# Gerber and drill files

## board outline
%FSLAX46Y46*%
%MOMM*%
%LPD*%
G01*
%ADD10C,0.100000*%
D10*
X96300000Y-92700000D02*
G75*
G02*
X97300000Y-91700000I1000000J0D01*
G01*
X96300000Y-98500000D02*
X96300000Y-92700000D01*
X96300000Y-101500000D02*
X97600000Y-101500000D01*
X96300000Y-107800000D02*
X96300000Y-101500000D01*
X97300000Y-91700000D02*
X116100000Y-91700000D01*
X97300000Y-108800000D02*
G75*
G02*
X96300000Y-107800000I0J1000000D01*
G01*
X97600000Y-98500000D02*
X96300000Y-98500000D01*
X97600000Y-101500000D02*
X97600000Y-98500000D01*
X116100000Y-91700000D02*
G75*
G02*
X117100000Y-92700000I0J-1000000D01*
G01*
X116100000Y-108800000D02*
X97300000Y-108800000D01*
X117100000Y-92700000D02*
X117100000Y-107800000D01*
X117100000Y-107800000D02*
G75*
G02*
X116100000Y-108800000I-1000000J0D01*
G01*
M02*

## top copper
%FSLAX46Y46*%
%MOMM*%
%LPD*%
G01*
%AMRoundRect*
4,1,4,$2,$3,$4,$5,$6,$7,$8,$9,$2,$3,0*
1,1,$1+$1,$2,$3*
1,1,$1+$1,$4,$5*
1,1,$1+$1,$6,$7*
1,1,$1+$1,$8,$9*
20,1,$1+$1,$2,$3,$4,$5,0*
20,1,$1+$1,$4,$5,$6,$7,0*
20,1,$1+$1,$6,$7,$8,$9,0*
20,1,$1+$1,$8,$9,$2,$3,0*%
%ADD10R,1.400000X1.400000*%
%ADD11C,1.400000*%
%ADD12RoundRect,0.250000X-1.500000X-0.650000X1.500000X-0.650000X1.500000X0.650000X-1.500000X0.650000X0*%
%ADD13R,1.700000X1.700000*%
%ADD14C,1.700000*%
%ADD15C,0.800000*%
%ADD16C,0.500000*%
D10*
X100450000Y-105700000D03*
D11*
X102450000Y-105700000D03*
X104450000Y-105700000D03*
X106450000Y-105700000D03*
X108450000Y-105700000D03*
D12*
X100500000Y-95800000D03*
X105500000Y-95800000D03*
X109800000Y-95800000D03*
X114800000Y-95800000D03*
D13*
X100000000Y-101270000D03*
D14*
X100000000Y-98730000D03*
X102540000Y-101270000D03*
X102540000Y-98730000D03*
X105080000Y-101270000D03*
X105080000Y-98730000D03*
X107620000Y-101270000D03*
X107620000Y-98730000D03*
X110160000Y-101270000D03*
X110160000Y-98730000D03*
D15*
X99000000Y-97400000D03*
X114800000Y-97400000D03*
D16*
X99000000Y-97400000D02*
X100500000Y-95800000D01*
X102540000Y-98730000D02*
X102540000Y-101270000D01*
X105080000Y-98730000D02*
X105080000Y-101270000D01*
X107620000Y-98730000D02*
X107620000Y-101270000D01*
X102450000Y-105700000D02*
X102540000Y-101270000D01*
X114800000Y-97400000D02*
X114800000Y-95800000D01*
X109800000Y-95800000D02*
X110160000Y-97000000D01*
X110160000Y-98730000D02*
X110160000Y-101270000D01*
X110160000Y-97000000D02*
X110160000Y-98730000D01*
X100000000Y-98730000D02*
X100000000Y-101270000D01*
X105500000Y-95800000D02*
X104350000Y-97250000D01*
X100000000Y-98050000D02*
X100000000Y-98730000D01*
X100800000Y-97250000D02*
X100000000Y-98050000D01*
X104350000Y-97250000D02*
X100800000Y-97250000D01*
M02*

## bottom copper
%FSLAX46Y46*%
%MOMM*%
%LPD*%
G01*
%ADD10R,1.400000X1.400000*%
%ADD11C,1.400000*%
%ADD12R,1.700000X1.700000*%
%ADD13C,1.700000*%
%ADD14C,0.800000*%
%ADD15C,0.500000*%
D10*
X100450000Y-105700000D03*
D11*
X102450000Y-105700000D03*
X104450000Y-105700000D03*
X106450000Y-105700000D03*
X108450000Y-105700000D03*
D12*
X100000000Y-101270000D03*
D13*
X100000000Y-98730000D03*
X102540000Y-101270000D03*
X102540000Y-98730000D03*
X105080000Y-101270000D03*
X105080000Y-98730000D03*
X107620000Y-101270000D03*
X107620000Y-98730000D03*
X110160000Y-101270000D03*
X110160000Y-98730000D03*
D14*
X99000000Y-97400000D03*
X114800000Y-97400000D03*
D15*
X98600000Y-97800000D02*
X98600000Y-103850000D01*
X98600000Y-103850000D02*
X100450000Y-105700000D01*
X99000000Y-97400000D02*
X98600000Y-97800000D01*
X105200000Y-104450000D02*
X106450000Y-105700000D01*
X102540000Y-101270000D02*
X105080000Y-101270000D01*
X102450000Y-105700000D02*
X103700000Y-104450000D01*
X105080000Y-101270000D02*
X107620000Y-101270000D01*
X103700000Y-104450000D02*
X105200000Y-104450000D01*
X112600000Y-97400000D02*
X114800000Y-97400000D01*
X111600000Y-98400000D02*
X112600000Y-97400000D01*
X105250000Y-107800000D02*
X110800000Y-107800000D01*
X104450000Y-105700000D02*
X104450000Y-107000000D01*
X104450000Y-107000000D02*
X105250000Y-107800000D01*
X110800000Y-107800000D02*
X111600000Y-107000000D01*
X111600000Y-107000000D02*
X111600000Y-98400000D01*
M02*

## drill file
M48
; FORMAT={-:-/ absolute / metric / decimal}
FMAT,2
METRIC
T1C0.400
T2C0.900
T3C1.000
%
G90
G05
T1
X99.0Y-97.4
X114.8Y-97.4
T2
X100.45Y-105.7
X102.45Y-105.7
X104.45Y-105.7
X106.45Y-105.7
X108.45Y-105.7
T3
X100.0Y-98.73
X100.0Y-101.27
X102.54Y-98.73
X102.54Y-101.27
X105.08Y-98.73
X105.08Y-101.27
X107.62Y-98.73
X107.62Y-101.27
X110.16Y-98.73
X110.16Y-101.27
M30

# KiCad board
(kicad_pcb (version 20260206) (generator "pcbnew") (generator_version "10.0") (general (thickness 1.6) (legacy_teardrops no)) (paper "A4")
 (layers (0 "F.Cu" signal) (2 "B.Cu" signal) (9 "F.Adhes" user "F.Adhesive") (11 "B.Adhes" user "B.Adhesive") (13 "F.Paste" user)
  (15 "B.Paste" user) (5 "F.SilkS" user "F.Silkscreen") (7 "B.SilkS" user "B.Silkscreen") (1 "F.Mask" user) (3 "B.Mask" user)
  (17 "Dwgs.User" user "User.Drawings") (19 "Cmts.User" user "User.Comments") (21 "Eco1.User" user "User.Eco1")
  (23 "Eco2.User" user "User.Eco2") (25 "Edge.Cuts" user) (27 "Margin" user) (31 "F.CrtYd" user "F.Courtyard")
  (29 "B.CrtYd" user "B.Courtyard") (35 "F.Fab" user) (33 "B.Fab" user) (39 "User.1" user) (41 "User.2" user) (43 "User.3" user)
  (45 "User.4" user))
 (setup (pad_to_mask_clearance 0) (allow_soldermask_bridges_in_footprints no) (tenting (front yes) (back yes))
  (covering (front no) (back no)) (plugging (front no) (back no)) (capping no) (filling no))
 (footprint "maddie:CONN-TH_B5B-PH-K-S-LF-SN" (layer "F.Cu") (at 104.45 105.7 180)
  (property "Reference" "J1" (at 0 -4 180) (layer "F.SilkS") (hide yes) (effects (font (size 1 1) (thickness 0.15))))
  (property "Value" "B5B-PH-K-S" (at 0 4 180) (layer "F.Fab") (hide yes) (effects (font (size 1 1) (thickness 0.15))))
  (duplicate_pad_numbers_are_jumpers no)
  (pad "1" thru_hole rect (at 4 0 180) (size 1.4 1.4) (drill 0.900024) (layers "*.Cu" "*.Mask") (remove_unused_layers no) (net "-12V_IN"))
  (pad "2" thru_hole circle (at 2 0 180) (size 1.4 1.4) (drill 0.900024) (layers "*.Cu" "*.Mask") (remove_unused_layers no) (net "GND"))
  (pad "3" thru_hole circle (at 0 0 180) (size 1.4 1.4) (drill 0.900024) (layers "*.Cu" "*.Mask") (remove_unused_layers no) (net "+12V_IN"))
  (pad "4" thru_hole circle (at -2 0 180) (size 1.4 1.4) (drill 0.900024) (layers "*.Cu" "*.Mask") (remove_unused_layers no) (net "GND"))
  (pad "5" thru_hole circle (at -4 0 180) (size 1.4 1.4) (drill 0.900024) (layers "*.Cu" "*.Mask") (remove_unused_layers no)
   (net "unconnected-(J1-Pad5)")))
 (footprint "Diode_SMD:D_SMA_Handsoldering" (layer "F.Cu") (at 103 95.8)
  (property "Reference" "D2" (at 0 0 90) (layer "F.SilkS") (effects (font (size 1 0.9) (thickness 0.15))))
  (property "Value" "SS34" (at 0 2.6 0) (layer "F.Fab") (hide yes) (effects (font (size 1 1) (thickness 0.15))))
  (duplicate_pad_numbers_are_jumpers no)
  (pad "1" smd roundrect (at -2.5 0) (size 3.5 1.8) (layers "F.Cu" "F.Mask" "F.Paste") (roundrect_rratio 0.1388888889) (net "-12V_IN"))
  (pad "2" smd roundrect (at 2.5 0) (size 3.5 1.8) (layers "F.Cu" "F.Mask" "F.Paste") (roundrect_rratio 0.1388888889) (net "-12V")))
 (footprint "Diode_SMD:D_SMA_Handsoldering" (layer "F.Cu") (at 112.3 95.8)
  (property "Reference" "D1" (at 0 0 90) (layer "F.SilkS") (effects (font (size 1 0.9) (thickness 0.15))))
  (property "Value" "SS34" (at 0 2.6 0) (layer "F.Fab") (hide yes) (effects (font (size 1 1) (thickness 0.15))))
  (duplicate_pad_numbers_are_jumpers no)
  (pad "1" smd roundrect (at -2.5 0) (size 3.5 1.8) (layers "F.Cu" "F.Mask" "F.Paste") (roundrect_rratio 0.1388888889) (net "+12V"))
  (pad "2" smd roundrect (at 2.5 0) (size 3.5 1.8) (layers "F.Cu" "F.Mask" "F.Paste") (roundrect_rratio 0.1388888889) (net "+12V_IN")))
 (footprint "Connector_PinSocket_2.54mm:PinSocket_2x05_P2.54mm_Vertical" (layer "B.Cu") (at 100 101.27 -90)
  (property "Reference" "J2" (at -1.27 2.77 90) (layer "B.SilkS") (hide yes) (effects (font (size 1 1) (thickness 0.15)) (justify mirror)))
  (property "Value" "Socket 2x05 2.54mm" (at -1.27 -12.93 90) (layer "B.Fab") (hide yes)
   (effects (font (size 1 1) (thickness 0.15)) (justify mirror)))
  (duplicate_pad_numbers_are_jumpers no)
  (pad "1" thru_hole rect (at 0 0 270) (size 1.7 1.7) (drill 1) (layers "*.Cu" "*.Mask") (remove_unused_layers no) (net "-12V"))
  (pad "2" thru_hole circle (at -2.54 0 270) (size 1.7 1.7) (drill 1) (layers "*.Cu" "*.Mask") (remove_unused_layers no) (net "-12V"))
  (pad "3" thru_hole circle (at 0 -2.54 270) (size 1.7 1.7) (drill 1) (layers "*.Cu" "*.Mask") (remove_unused_layers no) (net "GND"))
  (pad "4" thru_hole circle (at -2.54 -2.54 270) (size 1.7 1.7) (drill 1) (layers "*.Cu" "*.Mask") (remove_unused_layers no) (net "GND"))
  (pad "5" thru_hole circle (at 0 -5.08 270) (size 1.7 1.7) (drill 1) (layers "*.Cu" "*.Mask") (remove_unused_layers no) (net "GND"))
  (pad "6" thru_hole circle (at -2.54 -5.08 270) (size 1.7 1.7) (drill 1) (layers "*.Cu" "*.Mask") (remove_unused_layers no) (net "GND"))
  (pad "7" thru_hole circle (at 0 -7.62 270) (size 1.7 1.7) (drill 1) (layers "*.Cu" "*.Mask") (remove_unused_layers no) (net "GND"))
  (pad "8" thru_hole circle (at -2.54 -7.62 270) (size 1.7 1.7) (drill 1) (layers "*.Cu" "*.Mask") (remove_unused_layers no) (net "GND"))
  (pad "9" thru_hole circle (at 0 -10.16 270) (size 1.7 1.7) (drill 1) (layers "*.Cu" "*.Mask") (remove_unused_layers no) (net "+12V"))
  (pad "10" thru_hole circle (at -2.54 -10.16 270) (size 1.7 1.7) (drill 1) (layers "*.Cu" "*.Mask") (remove_unused_layers no) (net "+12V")))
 (gr_arc (start 96.3 92.7) (mid 96.59289 91.99289) (end 97.3 91.7) (stroke (width 0.1) (type default)) (layer "Edge.Cuts"))
 (gr_line (start 96.3 98.5) (end 96.3 92.7) (stroke (width 0.1) (type default)) (layer "Edge.Cuts"))
 (gr_line (start 96.3 101.5) (end 97.6 101.5) (stroke (width 0.1) (type default)) (layer "Edge.Cuts"))
 (gr_line (start 96.3 107.8) (end 96.3 101.5) (stroke (width 0.1) (type default)) (layer "Edge.Cuts"))
 (gr_line (start 97.3 91.7) (end 116.1 91.7) (stroke (width 0.1) (type default)) (layer "Edge.Cuts"))
 (gr_arc (start 97.3 108.8) (mid 96.59289 108.50711) (end 96.3 107.8) (stroke (width 0.1) (type default)) (layer "Edge.Cuts"))
 (gr_line (start 97.6 98.5) (end 96.3 98.5) (stroke (width 0.1) (type default)) (layer "Edge.Cuts"))
 (gr_line (start 97.6 101.5) (end 97.6 98.5) (stroke (width 0.1) (type default)) (layer "Edge.Cuts"))
 (gr_arc (start 116.1 91.7) (mid 116.80711 91.99289) (end 117.1 92.7) (stroke (width 0.1) (type default)) (layer "Edge.Cuts"))
 (gr_line (start 116.1 108.8) (end 97.3 108.8) (stroke (width 0.1) (type default)) (layer "Edge.Cuts"))
 (gr_line (start 117.1 92.7) (end 117.1 107.8) (stroke (width 0.1) (type default)) (layer "Edge.Cuts"))
 (gr_arc (start 117.1 107.8) (mid 116.80711 108.50711) (end 116.1 108.8) (stroke (width 0.1) (type default)) (layer "Edge.Cuts"))
 (segment (start 99 97.4) (end 100.5 95.8) (width 0.5) (layer "F.Cu") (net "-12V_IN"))
 (via (at 99 97.4) (size 0.8) (drill 0.4) (layers "F.Cu" "B.Cu") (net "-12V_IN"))
 (segment (start 98.6 97.8) (end 98.6 103.85) (width 0.5) (layer "B.Cu") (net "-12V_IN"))
 (segment (start 98.6 103.85) (end 100.45 105.7) (width 0.5) (layer "B.Cu") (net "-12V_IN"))
 (segment (start 99 97.4) (end 98.6 97.8) (width 0.5) (layer "B.Cu") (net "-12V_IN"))
 (segment (start 102.54 98.73) (end 102.54 101.27) (width 0.5) (layer "F.Cu") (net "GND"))
 (segment (start 105.08 98.73) (end 105.08 101.27) (width 0.5) (layer "F.Cu") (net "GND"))
 (segment (start 107.62 98.73) (end 107.62 101.27) (width 0.5) (layer "F.Cu") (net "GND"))
 (segment (start 102.45 105.7) (end 102.54 101.27) (width 0.5) (layer "F.Cu") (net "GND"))
 (segment (start 105.2 104.45) (end 106.45 105.7) (width 0.5) (layer "B.Cu") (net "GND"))
 (segment (start 102.54 101.27) (end 105.08 101.27) (width 0.5) (layer "B.Cu") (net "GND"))
 (segment (start 102.45 105.7) (end 103.7 104.45) (width 0.5) (layer "B.Cu") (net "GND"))
 (segment (start 105.08 101.27) (end 107.62 101.27) (width 0.5) (layer "B.Cu") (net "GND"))
 (segment (start 103.7 104.45) (end 105.2 104.45) (width 0.5) (layer "B.Cu") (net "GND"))
 (segment (start 114.8 97.4) (end 114.8 95.8) (width 0.5) (layer "F.Cu") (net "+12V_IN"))
 (via (at 114.8 97.4) (size 0.8) (drill 0.4) (layers "F.Cu" "B.Cu") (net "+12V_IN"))
 (segment (start 112.6 97.4) (end 114.8 97.4) (width 0.5) (layer "B.Cu") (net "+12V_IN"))
 (segment (start 111.6 98.4) (end 112.6 97.4) (width 0.5) (layer "B.Cu") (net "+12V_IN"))
 (segment (start 105.25 107.8) (end 110.8 107.8) (width 0.5) (layer "B.Cu") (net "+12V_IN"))
 (segment (start 104.45 105.7) (end 104.45 107) (width 0.5) (layer "B.Cu") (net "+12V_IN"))
 (segment (start 104.45 107) (end 105.25 107.8) (width 0.5) (layer "B.Cu") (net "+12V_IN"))
 (segment (start 110.8 107.8) (end 111.6 107) (width 0.5) (layer "B.Cu") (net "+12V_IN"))
 (segment (start 111.6 107) (end 111.6 98.4) (width 0.5) (layer "B.Cu") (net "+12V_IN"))
 (segment (start 109.8 95.8) (end 110.16 97) (width 0.5) (layer "F.Cu") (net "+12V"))
 (segment (start 110.16 98.73) (end 110.16 101.27) (width 0.5) (layer "F.Cu") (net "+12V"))
 (segment (start 110.16 97) (end 110.16 98.73) (width 0.5) (layer "F.Cu") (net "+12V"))
 (segment (start 100 98.73) (end 100 101.27) (width 0.5) (layer "F.Cu") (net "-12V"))
 (segment (start 105.5 95.8) (end 104.35 97.25) (width 0.5) (layer "F.Cu") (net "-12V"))
 (segment (start 100 98.05) (end 100 98.73) (width 0.5) (layer "F.Cu") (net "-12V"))
 (segment (start 100.8 97.25) (end 100 98.05) (width 0.5) (layer "F.Cu") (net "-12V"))
 (segment (start 104.35 97.25) (end 100.8 97.25) (width 0.5) (layer "F.Cu") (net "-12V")))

